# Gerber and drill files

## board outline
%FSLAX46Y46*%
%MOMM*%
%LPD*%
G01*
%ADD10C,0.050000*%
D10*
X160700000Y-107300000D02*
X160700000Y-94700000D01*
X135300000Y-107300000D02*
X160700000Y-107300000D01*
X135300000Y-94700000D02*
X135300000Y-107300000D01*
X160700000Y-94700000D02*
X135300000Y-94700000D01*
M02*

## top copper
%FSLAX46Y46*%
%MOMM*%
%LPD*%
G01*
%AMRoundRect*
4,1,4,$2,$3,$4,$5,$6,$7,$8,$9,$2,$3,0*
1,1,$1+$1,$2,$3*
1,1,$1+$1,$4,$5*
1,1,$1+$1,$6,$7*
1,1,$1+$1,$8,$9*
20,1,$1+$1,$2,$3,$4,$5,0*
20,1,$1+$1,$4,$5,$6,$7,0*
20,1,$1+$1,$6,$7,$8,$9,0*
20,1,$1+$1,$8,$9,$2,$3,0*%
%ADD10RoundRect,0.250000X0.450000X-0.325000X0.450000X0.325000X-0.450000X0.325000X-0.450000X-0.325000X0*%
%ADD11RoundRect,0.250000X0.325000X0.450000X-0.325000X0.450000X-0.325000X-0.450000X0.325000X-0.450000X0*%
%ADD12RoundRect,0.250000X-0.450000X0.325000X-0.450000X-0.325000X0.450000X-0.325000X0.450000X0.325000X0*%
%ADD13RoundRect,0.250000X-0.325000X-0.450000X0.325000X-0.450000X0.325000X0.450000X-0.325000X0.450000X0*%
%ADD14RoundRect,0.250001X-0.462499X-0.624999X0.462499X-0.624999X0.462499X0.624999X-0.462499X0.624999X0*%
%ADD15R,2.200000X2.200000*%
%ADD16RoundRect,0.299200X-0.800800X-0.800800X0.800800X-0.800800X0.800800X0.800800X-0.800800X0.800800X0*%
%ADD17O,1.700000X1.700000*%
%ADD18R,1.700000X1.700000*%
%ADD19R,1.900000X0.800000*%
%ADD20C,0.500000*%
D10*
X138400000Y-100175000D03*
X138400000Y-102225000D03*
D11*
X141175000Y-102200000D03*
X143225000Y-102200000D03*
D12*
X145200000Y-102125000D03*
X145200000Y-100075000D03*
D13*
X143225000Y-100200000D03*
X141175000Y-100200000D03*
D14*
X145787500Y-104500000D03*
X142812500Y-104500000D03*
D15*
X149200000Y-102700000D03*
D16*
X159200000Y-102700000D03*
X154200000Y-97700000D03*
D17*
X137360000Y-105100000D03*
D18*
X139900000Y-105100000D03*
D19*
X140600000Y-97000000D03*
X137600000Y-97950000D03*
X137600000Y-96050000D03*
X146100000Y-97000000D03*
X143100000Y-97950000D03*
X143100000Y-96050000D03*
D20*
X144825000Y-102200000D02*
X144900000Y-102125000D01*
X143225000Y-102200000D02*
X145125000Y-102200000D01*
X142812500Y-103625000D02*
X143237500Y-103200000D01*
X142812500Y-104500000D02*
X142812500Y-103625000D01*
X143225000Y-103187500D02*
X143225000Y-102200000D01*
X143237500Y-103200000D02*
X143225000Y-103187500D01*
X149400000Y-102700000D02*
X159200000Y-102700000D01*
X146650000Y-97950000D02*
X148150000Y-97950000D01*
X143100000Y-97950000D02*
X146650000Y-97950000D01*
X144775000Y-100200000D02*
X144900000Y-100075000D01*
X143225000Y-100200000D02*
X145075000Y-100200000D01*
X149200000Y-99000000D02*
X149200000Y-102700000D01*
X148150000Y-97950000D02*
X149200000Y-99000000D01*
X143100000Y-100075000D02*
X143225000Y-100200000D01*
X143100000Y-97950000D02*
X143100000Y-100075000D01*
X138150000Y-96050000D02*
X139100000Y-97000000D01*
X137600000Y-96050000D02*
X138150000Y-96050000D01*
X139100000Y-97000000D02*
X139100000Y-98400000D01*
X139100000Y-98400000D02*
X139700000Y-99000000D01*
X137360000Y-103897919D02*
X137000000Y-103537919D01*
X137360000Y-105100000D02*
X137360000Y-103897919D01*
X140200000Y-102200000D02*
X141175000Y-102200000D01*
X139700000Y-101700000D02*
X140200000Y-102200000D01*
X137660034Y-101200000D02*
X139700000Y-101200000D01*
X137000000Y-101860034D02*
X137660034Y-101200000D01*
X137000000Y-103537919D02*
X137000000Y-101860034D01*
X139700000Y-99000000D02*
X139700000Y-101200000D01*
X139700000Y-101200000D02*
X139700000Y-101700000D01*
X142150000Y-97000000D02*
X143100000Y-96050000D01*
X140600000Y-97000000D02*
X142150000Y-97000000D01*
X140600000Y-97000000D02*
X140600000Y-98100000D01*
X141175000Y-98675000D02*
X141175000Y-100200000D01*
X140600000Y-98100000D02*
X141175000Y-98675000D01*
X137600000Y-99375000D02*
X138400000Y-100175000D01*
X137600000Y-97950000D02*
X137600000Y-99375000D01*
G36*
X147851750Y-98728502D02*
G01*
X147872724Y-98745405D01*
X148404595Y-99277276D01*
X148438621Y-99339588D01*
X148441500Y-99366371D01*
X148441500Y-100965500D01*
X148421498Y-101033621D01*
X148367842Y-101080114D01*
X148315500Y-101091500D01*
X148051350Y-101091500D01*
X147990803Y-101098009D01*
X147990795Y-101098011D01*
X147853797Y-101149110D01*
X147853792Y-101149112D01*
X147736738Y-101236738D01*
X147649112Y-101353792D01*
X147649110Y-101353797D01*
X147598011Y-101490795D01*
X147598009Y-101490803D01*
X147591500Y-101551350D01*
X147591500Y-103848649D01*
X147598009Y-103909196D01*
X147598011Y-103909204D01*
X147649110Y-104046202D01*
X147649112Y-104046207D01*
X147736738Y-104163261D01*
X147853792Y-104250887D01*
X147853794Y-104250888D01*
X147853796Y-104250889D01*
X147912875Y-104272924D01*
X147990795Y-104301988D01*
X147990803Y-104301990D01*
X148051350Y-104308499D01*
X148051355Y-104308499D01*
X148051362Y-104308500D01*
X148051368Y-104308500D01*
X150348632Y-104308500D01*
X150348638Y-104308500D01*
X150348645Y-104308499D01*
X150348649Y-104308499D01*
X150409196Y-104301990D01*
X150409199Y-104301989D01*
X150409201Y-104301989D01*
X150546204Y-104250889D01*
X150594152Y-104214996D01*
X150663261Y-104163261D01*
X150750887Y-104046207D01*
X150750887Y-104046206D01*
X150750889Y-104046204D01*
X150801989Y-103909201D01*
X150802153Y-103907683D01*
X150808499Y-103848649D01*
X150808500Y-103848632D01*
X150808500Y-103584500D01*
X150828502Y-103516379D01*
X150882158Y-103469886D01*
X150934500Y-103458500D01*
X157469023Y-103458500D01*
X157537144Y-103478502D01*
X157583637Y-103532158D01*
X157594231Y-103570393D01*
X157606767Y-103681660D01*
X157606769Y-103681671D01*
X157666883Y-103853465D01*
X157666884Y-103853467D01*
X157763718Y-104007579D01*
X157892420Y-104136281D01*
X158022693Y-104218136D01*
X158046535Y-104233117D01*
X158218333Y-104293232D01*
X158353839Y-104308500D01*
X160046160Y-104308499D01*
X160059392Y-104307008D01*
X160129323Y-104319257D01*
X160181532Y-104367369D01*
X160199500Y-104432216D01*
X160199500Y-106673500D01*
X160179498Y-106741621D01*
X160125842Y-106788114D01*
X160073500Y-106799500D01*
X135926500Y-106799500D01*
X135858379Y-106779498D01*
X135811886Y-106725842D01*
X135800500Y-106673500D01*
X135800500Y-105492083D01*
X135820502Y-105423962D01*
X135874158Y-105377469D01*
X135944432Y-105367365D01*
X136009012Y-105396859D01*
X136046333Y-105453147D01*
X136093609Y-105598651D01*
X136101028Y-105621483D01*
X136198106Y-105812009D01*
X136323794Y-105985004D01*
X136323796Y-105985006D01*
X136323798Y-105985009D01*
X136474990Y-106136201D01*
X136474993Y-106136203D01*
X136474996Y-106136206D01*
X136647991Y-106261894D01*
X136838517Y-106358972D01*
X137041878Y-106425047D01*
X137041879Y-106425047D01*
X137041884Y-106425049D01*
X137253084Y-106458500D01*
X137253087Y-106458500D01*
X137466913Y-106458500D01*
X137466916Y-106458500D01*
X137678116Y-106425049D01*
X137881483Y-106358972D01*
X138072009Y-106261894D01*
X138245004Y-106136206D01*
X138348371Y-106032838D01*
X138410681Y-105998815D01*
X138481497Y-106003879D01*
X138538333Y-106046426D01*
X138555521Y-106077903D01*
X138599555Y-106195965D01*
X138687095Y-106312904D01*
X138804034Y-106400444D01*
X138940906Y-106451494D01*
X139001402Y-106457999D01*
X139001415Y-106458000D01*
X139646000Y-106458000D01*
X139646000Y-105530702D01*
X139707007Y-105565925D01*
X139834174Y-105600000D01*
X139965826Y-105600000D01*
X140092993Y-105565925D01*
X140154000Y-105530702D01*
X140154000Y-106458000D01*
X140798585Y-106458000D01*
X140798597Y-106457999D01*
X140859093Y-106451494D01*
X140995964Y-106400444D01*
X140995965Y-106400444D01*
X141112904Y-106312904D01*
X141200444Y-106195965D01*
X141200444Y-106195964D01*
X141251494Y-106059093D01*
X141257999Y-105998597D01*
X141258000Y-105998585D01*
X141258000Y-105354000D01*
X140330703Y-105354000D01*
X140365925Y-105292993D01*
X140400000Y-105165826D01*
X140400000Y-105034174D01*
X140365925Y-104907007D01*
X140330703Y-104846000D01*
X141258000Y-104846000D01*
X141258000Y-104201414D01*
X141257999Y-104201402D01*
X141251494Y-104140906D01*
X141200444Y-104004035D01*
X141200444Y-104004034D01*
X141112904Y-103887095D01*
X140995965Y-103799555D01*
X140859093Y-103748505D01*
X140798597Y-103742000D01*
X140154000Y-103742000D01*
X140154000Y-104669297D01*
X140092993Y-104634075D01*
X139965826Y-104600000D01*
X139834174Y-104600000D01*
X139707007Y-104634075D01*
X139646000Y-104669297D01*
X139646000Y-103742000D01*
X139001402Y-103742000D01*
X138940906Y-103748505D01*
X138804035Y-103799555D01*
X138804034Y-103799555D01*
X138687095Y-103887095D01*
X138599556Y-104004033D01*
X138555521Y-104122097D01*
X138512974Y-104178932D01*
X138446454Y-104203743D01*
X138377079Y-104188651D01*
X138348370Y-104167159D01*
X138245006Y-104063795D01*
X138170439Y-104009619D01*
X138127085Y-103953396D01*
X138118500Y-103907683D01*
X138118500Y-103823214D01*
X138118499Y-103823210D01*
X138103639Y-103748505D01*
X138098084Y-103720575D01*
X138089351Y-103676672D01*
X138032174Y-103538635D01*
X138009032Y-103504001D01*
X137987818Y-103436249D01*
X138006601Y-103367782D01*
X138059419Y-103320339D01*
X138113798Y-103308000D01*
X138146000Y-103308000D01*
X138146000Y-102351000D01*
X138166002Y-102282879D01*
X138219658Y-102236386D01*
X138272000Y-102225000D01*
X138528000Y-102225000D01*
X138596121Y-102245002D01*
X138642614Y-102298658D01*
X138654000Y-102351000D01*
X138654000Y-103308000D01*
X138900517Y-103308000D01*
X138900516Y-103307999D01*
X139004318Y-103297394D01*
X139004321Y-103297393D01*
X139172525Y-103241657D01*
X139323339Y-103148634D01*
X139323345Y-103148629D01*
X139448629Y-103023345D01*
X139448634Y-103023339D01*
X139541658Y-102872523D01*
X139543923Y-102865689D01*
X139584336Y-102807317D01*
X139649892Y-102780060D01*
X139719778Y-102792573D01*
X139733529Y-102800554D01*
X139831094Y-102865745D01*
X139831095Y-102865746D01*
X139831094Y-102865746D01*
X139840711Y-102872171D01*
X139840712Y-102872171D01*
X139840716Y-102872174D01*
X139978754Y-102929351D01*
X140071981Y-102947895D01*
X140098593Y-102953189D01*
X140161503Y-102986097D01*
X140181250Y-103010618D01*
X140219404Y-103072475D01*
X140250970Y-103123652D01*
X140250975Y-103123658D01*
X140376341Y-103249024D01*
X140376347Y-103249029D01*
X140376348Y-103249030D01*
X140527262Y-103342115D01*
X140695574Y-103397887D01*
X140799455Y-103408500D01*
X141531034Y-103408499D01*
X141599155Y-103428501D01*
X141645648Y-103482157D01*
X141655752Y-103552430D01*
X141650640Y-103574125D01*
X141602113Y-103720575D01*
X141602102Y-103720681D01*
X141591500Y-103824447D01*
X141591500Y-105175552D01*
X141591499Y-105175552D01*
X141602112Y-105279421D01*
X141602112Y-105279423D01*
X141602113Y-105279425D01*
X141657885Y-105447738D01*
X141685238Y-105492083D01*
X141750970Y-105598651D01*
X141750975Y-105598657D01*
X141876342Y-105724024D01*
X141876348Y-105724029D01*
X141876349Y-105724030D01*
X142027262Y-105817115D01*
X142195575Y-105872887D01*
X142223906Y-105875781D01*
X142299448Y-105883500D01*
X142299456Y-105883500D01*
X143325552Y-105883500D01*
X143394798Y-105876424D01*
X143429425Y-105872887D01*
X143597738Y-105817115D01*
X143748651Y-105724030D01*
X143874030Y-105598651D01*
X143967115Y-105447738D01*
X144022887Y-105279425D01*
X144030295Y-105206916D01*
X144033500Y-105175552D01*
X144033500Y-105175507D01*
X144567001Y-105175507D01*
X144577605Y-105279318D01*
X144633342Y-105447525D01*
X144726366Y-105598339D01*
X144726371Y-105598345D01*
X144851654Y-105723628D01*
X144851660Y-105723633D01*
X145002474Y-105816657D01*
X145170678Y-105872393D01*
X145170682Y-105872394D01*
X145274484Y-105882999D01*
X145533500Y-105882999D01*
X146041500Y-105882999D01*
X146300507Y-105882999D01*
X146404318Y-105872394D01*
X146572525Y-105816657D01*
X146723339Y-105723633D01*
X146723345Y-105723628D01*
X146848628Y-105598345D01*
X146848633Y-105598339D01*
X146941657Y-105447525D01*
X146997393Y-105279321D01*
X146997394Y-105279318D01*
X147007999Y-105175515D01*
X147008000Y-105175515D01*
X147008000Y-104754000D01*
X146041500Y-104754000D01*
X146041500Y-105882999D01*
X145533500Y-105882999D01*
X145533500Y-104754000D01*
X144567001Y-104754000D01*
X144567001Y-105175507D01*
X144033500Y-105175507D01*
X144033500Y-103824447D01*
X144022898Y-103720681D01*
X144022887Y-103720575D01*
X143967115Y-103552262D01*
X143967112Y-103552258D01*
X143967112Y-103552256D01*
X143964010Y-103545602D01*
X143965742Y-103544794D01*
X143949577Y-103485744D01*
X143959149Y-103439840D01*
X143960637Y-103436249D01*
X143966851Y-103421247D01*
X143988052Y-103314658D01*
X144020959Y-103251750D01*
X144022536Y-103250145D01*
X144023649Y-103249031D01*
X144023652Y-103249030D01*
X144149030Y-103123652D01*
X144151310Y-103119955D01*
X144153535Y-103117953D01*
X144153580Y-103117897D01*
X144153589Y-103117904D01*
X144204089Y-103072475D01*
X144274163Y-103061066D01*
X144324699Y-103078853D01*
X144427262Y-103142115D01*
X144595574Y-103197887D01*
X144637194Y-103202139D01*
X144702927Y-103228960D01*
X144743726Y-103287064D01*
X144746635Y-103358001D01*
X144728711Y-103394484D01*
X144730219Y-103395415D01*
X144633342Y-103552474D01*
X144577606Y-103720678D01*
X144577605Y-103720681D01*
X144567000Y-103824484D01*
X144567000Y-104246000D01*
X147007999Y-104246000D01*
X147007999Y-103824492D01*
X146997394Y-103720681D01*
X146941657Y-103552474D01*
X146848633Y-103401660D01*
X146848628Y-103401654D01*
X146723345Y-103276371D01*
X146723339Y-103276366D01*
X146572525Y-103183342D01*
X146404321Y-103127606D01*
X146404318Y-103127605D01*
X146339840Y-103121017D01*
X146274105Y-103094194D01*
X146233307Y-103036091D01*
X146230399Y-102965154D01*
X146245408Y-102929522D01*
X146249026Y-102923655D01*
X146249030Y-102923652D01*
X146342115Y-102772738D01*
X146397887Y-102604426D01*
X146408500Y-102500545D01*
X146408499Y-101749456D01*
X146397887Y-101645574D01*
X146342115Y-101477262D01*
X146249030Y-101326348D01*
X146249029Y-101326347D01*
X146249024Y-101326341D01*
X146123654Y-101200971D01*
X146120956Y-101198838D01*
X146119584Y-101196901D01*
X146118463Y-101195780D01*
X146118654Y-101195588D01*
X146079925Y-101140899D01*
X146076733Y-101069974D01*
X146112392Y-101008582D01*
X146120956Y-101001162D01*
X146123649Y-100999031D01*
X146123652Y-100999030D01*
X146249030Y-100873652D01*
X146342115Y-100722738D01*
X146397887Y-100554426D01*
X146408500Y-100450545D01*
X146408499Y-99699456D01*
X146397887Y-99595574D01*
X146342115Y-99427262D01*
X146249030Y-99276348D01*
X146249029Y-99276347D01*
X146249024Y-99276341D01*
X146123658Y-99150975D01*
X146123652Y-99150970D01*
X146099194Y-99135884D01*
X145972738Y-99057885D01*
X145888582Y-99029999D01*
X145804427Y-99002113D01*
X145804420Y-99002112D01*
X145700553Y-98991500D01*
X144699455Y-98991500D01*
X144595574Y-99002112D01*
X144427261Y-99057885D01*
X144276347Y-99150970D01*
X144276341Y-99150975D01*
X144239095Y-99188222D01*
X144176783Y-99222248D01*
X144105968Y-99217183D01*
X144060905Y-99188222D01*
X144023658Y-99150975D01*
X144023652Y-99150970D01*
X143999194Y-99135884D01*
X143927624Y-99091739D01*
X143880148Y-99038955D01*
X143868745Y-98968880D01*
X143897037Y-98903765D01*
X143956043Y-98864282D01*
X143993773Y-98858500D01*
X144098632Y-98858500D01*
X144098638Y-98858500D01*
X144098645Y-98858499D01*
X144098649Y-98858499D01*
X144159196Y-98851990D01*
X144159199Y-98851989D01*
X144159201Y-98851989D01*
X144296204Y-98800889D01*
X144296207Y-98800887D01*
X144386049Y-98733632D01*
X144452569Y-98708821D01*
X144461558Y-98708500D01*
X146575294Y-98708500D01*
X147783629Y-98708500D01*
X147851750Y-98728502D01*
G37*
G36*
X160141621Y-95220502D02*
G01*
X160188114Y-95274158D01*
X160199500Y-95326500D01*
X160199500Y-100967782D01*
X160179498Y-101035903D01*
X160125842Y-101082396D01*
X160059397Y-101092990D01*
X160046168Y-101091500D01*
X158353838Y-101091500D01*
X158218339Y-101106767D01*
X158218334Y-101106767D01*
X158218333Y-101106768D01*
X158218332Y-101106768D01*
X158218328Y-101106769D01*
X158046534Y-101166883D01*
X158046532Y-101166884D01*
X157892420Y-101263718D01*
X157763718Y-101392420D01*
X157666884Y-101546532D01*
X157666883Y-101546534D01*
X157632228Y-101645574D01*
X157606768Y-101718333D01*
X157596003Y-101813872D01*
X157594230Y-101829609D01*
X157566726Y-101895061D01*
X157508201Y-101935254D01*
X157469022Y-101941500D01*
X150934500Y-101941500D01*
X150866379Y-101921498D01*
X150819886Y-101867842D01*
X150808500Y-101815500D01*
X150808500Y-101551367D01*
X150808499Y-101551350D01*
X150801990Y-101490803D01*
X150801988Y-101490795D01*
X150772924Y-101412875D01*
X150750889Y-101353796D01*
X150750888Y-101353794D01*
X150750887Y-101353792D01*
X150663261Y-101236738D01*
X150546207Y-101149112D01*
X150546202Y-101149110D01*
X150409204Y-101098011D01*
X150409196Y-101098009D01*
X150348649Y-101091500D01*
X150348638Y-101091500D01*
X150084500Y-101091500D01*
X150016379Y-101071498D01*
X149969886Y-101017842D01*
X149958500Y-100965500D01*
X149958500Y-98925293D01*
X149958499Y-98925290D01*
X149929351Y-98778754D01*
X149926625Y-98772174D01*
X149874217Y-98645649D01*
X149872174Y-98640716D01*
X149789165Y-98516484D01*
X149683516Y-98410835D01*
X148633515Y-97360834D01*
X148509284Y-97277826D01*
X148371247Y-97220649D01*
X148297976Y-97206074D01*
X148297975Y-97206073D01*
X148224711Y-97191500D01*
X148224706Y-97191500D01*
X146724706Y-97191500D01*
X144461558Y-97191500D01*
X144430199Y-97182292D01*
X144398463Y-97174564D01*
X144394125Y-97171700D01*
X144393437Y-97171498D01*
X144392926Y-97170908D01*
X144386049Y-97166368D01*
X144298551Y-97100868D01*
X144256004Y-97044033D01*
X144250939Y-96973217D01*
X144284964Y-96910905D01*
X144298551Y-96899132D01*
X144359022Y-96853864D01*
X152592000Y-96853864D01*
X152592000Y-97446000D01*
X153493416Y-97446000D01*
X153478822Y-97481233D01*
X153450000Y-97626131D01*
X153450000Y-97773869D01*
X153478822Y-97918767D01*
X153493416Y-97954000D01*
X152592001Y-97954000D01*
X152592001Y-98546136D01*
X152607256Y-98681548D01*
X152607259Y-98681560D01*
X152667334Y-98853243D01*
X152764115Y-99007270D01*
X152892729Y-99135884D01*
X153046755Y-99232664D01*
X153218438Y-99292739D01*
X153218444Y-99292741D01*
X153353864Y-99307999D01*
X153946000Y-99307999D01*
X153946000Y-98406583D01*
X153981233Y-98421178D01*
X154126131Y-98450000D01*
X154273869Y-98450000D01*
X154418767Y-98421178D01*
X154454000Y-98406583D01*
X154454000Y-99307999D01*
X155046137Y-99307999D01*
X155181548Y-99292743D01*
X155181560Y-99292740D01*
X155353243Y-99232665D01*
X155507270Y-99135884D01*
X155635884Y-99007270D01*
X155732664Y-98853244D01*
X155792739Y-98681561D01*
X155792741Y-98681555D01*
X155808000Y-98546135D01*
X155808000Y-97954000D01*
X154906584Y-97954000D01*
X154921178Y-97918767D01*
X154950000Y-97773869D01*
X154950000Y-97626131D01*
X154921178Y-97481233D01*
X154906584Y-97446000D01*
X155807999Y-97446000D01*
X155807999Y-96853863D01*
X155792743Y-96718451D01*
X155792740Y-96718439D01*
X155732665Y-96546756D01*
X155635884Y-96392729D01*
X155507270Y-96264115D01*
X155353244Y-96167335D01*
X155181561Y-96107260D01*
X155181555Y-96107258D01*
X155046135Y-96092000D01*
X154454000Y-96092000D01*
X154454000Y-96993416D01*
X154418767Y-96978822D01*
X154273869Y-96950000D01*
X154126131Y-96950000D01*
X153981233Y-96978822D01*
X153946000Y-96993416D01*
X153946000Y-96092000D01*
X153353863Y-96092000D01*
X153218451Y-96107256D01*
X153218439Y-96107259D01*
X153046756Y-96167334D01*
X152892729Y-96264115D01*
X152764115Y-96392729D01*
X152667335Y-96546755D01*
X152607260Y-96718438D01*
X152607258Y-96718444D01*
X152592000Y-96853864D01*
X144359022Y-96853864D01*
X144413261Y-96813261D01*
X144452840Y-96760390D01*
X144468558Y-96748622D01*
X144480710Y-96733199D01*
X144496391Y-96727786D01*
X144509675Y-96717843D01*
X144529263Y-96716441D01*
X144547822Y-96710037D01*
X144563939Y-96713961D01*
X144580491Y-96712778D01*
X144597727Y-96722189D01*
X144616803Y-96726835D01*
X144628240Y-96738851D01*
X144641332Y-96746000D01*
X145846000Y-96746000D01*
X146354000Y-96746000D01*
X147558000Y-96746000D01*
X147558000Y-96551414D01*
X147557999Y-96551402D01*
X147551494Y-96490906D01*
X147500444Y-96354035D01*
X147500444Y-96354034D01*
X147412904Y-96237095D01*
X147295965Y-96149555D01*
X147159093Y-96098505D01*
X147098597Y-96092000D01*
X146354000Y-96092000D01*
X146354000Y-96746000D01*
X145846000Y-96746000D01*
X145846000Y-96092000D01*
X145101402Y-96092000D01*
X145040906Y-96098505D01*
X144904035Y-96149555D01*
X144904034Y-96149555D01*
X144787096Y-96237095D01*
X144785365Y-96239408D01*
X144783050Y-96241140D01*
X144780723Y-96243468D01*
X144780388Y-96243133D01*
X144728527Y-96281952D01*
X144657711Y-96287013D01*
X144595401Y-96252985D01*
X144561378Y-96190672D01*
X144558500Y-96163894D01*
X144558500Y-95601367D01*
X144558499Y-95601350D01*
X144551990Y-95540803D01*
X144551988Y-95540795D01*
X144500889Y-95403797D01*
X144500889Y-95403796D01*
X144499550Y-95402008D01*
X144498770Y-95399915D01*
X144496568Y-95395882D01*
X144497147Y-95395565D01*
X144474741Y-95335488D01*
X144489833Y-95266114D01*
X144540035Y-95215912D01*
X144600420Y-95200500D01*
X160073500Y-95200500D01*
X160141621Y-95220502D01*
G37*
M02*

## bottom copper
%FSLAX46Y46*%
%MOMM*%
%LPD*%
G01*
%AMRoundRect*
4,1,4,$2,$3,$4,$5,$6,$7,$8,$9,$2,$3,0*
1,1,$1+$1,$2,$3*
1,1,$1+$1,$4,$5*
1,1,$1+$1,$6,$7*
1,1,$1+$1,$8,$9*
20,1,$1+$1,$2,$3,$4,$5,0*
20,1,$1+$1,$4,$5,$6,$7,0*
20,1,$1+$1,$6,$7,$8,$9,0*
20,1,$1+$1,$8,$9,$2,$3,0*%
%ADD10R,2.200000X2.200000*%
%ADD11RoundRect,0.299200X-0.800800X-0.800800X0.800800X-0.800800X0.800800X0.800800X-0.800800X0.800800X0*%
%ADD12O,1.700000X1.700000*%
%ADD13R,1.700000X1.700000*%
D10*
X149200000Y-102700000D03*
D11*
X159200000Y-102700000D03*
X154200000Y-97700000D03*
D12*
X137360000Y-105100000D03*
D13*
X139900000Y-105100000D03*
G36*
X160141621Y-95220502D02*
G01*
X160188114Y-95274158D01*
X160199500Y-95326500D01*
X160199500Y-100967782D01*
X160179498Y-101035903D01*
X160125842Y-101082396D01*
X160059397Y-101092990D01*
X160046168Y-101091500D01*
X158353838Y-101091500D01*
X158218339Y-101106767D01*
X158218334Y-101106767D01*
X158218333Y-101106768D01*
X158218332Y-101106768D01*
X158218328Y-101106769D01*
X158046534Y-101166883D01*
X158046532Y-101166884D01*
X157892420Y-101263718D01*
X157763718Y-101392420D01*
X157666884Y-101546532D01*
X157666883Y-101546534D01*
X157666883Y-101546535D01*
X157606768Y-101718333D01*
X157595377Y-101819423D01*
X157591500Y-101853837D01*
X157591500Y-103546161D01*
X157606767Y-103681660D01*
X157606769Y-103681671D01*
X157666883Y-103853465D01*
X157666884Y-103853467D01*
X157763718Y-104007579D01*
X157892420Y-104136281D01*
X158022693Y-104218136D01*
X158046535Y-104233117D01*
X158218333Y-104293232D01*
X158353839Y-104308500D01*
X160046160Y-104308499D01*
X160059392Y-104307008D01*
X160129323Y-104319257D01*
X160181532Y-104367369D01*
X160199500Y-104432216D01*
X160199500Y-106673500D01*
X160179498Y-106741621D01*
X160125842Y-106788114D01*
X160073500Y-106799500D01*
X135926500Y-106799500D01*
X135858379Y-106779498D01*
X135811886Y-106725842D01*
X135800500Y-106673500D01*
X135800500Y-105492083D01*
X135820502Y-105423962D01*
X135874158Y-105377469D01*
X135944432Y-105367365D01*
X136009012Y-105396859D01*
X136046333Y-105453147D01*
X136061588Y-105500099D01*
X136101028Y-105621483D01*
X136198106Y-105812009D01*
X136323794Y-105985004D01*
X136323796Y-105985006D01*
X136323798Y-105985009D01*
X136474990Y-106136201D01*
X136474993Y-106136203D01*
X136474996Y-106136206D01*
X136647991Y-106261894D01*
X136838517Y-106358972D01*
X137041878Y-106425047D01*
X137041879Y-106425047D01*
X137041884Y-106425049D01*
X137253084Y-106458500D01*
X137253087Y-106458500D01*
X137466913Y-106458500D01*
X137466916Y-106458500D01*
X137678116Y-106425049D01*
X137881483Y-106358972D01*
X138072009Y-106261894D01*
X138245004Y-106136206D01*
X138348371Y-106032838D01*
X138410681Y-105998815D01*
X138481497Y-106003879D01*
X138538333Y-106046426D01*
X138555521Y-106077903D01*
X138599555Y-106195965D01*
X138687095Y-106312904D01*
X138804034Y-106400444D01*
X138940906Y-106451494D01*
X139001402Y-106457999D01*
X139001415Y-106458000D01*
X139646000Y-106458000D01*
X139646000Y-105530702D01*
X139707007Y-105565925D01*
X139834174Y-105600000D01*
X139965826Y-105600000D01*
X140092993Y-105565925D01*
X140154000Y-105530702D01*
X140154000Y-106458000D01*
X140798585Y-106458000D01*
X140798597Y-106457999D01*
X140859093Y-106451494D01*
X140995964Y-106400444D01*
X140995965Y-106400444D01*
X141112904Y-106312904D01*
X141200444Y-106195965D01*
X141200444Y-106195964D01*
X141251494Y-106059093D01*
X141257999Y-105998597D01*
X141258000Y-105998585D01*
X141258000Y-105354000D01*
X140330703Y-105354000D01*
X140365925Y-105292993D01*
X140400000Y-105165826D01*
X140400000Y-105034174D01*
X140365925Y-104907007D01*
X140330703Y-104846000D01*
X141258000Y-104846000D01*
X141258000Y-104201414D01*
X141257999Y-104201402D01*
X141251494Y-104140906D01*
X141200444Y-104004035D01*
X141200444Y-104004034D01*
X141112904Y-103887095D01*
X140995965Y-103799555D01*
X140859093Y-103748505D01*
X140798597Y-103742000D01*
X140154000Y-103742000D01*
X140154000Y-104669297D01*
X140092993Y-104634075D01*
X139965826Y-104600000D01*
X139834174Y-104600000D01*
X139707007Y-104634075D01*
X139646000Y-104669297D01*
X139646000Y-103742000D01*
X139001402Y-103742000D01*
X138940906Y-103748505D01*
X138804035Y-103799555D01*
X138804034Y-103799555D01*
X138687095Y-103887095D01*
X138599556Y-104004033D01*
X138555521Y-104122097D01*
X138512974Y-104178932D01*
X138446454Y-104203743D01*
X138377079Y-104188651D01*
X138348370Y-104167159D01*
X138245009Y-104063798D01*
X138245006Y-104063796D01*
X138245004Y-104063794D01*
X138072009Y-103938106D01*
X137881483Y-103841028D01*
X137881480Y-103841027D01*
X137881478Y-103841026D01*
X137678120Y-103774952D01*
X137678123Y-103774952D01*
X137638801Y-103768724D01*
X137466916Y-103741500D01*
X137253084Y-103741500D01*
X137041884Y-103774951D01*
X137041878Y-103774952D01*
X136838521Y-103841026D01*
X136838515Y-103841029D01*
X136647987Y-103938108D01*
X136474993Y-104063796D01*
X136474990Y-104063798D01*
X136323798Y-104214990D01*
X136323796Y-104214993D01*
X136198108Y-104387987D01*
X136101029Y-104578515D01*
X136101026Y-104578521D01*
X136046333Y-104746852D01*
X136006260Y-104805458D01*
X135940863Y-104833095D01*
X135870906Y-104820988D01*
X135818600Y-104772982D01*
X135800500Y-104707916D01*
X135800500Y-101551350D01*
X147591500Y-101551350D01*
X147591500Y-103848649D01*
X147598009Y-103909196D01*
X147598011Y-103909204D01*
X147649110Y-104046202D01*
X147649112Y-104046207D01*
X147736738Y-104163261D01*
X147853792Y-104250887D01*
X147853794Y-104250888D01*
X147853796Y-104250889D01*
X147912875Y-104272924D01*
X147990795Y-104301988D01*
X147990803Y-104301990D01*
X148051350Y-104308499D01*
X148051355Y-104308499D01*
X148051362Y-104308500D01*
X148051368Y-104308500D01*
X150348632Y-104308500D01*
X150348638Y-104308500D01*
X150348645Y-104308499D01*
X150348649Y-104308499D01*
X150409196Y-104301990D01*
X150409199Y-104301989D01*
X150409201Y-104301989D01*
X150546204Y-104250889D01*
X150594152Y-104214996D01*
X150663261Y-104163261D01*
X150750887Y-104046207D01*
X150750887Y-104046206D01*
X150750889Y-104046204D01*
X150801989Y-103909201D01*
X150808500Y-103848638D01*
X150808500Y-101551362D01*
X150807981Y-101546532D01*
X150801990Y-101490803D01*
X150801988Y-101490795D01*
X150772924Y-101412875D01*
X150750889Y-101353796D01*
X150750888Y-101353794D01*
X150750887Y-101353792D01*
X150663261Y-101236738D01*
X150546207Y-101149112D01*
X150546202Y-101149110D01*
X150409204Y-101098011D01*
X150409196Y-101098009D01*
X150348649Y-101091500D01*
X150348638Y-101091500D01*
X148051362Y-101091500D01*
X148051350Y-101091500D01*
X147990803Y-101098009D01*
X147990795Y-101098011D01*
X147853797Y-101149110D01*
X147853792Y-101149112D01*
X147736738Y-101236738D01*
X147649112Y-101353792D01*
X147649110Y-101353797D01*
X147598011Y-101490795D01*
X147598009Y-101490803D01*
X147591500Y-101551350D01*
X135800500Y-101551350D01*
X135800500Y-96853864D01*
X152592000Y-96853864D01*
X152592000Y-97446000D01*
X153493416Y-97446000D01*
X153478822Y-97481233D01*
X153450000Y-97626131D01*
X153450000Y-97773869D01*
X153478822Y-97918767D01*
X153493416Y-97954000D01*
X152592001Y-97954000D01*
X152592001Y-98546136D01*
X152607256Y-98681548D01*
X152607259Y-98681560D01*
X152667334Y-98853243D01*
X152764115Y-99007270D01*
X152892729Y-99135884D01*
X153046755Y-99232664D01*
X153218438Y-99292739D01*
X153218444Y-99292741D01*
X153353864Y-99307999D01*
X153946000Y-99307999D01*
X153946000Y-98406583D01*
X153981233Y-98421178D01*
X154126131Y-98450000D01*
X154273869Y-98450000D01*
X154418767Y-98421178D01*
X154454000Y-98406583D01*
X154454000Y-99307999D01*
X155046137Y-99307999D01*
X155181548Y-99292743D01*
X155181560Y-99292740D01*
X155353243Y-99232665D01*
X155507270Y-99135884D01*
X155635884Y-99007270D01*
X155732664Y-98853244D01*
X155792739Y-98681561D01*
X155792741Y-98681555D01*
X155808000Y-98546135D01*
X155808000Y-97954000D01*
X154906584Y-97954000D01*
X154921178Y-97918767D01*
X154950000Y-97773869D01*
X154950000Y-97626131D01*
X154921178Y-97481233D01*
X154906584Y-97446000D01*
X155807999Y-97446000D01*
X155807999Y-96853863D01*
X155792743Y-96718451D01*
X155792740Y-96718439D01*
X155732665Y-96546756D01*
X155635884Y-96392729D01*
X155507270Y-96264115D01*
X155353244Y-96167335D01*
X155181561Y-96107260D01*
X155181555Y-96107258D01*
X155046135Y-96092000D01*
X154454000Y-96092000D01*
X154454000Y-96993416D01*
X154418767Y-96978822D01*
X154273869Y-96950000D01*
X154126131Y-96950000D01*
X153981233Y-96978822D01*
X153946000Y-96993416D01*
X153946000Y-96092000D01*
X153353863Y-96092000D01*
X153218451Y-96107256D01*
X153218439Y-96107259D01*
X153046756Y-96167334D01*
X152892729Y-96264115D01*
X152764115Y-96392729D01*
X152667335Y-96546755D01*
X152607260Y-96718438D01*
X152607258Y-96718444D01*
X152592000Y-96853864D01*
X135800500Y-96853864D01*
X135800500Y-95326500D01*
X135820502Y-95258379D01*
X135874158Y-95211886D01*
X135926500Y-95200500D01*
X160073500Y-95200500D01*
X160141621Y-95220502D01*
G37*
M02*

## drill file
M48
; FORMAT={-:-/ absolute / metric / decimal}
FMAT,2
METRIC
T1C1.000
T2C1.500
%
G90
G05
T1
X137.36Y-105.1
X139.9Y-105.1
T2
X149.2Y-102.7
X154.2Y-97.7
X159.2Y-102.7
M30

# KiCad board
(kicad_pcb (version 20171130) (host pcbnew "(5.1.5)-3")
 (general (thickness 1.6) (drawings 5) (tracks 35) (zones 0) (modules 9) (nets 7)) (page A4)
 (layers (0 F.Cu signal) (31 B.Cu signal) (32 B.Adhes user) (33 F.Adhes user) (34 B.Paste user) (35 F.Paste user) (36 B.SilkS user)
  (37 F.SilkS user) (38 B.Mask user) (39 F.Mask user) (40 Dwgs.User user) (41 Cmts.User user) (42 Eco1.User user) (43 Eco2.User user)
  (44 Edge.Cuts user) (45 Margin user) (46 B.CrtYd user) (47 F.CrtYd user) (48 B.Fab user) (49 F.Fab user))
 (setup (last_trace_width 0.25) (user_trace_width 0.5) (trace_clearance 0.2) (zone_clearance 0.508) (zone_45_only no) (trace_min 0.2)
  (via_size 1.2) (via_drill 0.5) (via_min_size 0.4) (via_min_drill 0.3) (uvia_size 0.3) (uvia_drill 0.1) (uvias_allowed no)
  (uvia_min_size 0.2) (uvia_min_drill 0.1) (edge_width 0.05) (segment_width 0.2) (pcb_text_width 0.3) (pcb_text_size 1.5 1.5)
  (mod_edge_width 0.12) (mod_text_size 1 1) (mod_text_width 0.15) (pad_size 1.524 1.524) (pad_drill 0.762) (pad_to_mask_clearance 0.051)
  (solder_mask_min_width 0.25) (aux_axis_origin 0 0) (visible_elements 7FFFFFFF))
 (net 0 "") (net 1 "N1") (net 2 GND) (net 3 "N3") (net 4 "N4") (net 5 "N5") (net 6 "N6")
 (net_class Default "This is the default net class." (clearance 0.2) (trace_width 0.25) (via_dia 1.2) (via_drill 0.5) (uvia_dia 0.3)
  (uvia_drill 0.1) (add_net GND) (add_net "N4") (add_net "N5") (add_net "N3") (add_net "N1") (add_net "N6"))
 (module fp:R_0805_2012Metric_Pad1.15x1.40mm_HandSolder (layer F.Cu) (at 138.4 101.2 90)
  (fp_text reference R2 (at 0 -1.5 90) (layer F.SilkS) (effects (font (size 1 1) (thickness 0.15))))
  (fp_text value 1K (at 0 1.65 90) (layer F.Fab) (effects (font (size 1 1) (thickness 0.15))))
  (pad 2 smd roundrect (at 1.025 0 90) (size 1.15 1.4) (layers F.Cu F.Paste F.Mask) (roundrect_rratio 0.217391) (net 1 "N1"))
  (pad 1 smd roundrect (at -1.025 0 90) (size 1.15 1.4) (layers F.Cu F.Paste F.Mask) (roundrect_rratio 0.217391) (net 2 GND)))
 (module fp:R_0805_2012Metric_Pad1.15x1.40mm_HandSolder (layer F.Cu) (at 142.2 102.2 180)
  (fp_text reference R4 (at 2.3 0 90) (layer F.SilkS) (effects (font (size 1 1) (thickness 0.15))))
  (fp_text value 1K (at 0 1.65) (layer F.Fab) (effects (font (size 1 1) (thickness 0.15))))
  (pad 2 smd roundrect (at 1.025 0 180) (size 1.15 1.4) (layers F.Cu F.Paste F.Mask) (roundrect_rratio 0.217391) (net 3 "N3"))
  (pad 1 smd roundrect (at -1.025 0 180) (size 1.15 1.4) (layers F.Cu F.Paste F.Mask) (roundrect_rratio 0.217391) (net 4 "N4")))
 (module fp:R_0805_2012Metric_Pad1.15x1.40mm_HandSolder (layer F.Cu) (at 145.2 101.1 270)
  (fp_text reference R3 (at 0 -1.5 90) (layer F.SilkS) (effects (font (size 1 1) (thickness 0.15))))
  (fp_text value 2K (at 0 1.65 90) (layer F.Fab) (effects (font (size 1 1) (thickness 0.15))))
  (pad 2 smd roundrect (at 1.025 0 270) (size 1.15 1.4) (layers F.Cu F.Paste F.Mask) (roundrect_rratio 0.217391) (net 4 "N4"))
  (pad 1 smd roundrect (at -1.025 0 270) (size 1.15 1.4) (layers F.Cu F.Paste F.Mask) (roundrect_rratio 0.217391) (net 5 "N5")))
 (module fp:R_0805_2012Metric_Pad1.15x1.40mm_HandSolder (layer F.Cu) (at 142.2 100.2)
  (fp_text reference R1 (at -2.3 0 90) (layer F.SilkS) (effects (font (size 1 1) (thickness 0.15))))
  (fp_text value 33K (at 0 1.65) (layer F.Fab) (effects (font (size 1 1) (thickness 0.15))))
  (pad 2 smd roundrect (at 1.025 0) (size 1.15 1.4) (layers F.Cu F.Paste F.Mask) (roundrect_rratio 0.217391) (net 5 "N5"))
  (pad 1 smd roundrect (at -1.025 0) (size 1.15 1.4) (layers F.Cu F.Paste F.Mask) (roundrect_rratio 0.217391) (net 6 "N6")))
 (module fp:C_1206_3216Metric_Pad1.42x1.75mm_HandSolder (layer F.Cu) (at 144.3 104.5)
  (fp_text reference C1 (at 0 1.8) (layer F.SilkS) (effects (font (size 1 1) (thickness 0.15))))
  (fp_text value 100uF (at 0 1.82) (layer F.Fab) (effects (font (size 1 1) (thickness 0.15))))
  (pad 2 smd roundrect (at 1.4875 0) (size 1.425 1.75) (layers F.Cu F.Paste F.Mask) (roundrect_rratio 0.175439) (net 2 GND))
  (pad 1 smd roundrect (at -1.4875 0) (size 1.425 1.75) (layers F.Cu F.Paste F.Mask) (roundrect_rratio 0.175439) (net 4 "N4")))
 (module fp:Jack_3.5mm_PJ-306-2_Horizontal (layer F.Cu) (at 154.2 101.7)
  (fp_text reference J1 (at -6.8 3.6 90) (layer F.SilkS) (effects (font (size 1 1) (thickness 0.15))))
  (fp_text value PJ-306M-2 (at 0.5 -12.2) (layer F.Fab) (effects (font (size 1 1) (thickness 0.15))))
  (pad T thru_hole rect (at -5 1) (size 2.2 2.2) (drill 1.5) (layers *.Cu *.Mask) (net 5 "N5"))
  (pad R thru_hole roundrect (at 5 1) (size 2.2 2.2) (drill 1.5) (layers *.Cu *.Mask) (roundrect_rratio 0.136) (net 5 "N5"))
  (pad S thru_hole roundrect (at 0 -4) (size 2.2 2.2) (drill 1.5) (layers *.Cu *.Mask) (roundrect_rratio 0.136) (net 2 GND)))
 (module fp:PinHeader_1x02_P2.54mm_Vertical (layer F.Cu) (at 139.9 105.1 270)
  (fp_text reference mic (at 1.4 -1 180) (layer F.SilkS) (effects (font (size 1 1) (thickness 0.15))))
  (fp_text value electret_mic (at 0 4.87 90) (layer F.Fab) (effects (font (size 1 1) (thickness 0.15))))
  (pad 2 thru_hole oval (at 0 2.54 270) (size 1.7 1.7) (drill 1) (layers *.Cu *.Mask) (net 3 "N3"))
  (pad 1 thru_hole rect (at 0 0 270) (size 1.7 1.7) (drill 1) (layers *.Cu *.Mask) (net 2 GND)))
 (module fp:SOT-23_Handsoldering (layer F.Cu) (at 139.1 97)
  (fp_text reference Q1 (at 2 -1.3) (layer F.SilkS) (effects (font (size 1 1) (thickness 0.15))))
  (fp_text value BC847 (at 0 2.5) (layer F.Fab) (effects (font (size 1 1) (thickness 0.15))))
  (pad 3 smd rect (at 1.5 0) (size 1.9 0.8) (layers F.Cu F.Paste F.Mask) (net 6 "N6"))
  (pad 2 smd rect (at -1.5 0.95) (size 1.9 0.8) (layers F.Cu F.Paste F.Mask) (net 1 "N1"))
  (pad 1 smd rect (at -1.5 -0.95) (size 1.9 0.8) (layers F.Cu F.Paste F.Mask) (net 3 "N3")))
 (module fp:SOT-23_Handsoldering (layer F.Cu) (at 144.6 97)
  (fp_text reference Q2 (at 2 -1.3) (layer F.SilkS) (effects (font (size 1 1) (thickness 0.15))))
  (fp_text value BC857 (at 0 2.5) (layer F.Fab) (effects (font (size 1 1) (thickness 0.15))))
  (pad 3 smd rect (at 1.5 0) (size 1.9 0.8) (layers F.Cu F.Paste F.Mask) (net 2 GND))
  (pad 2 smd rect (at -1.5 0.95) (size 1.9 0.8) (layers F.Cu F.Paste F.Mask) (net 5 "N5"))
  (pad 1 smd rect (at -1.5 -0.95) (size 1.9 0.8) (layers F.Cu F.Paste F.Mask) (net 6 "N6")))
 (gr_line (start 160.7 107.3) (end 160.7 94.7) (layer Edge.Cuts) (width 0.05))
 (gr_line (start 135.3 107.3) (end 160.7 107.3) (layer Edge.Cuts) (width 0.05))
 (gr_line (start 135.3 94.7) (end 135.3 107.3) (layer Edge.Cuts) (width 0.05))
 (gr_line (start 160.7 94.7) (end 135.3 94.7) (layer Edge.Cuts) (width 0.05))
 (segment (start 144.825 102.2) (end 144.9 102.125) (width 0.5) (layer F.Cu) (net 4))
 (segment (start 143.225 102.2) (end 145.125 102.2) (width 0.5) (layer F.Cu) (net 4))
 (segment (start 142.8125 103.625) (end 143.2375 103.2) (width 0.5) (layer F.Cu) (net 4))
 (segment (start 142.8125 104.5) (end 142.8125 103.625) (width 0.5) (layer F.Cu) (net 4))
 (segment (start 143.225 103.1875) (end 143.225 102.2) (width 0.5) (layer F.Cu) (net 4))
 (segment (start 143.2375 103.2) (end 143.225 103.1875) (width 0.5) (layer F.Cu) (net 4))
 (segment (start 149.4 102.7) (end 159.2 102.7) (width 0.5) (layer F.Cu) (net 5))
 (segment (start 146.65 97.95) (end 148.15 97.95) (width 0.5) (layer F.Cu) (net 5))
 (segment (start 143.1 97.95) (end 146.65 97.95) (width 0.5) (layer F.Cu) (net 5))
 (segment (start 144.775 100.2) (end 144.9 100.075) (width 0.5) (layer F.Cu) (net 5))
 (segment (start 143.225 100.2) (end 145.075 100.2) (width 0.5) (layer F.Cu) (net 5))
 (segment (start 149.2 99) (end 149.2 102.7) (width 0.5) (layer F.Cu) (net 5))
 (segment (start 148.15 97.95) (end 149.2 99) (width 0.5) (layer F.Cu) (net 5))
 (segment (start 143.1 100.075) (end 143.225 100.2) (width 0.5) (layer F.Cu) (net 5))
 (segment (start 143.1 97.95) (end 143.1 100.075) (width 0.5) (layer F.Cu) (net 5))
 (segment (start 138.15 96.05) (end 139.1 97) (width 0.5) (layer F.Cu) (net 3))
 (segment (start 137.6 96.05) (end 138.15 96.05) (width 0.5) (layer F.Cu) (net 3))
 (segment (start 139.1 97) (end 139.1 98.4) (width 0.5) (layer F.Cu) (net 3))
 (segment (start 139.1 98.4) (end 139.7 99) (width 0.5) (layer F.Cu) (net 3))
 (segment (start 137.36 103.897919) (end 137 103.537919) (width 0.5) (layer F.Cu) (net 3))
 (segment (start 137.36 105.1) (end 137.36 103.897919) (width 0.5) (layer F.Cu) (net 3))
 (segment (start 140.2 102.2) (end 141.175 102.2) (width 0.5) (layer F.Cu) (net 3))
 (segment (start 139.7 101.7) (end 140.2 102.2) (width 0.5) (layer F.Cu) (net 3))
 (segment (start 137.660034 101.2) (end 139.7 101.2) (width 0.5) (layer F.Cu) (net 3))
 (segment (start 137 101.860034) (end 137.660034 101.2) (width 0.5) (layer F.Cu) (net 3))
 (segment (start 137 103.537919) (end 137 101.860034) (width 0.5) (layer F.Cu) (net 3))
 (segment (start 139.7 99) (end 139.7 101.2) (width 0.5) (layer F.Cu) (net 3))
 (segment (start 139.7 101.2) (end 139.7 101.7) (width 0.5) (layer F.Cu) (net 3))
 (segment (start 142.15 97) (end 143.1 96.05) (width 0.5) (layer F.Cu) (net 6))
 (segment (start 140.6 97) (end 142.15 97) (width 0.5) (layer F.Cu) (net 6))
 (segment (start 140.6 97) (end 140.6 98.1) (width 0.5) (layer F.Cu) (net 6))
 (segment (start 141.175 98.675) (end 141.175 100.2) (width 0.5) (layer F.Cu) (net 6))
 (segment (start 140.6 98.1) (end 141.175 98.675) (width 0.5) (layer F.Cu) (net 6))
 (segment (start 137.6 99.375) (end 138.4 100.175) (width 0.5) (layer F.Cu) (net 1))
 (segment (start 137.6 97.95) (end 137.6 99.375) (width 0.5) (layer F.Cu) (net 1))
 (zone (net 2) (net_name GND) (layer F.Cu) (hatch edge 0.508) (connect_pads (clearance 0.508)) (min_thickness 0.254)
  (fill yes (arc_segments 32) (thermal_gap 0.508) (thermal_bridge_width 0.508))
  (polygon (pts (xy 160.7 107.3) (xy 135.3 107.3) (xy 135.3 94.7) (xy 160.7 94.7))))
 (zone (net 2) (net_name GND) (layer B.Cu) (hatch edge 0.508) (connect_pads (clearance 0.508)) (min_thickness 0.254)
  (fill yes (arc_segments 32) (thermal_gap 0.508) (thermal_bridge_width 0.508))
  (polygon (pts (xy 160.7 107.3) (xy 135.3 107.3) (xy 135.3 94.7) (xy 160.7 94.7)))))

